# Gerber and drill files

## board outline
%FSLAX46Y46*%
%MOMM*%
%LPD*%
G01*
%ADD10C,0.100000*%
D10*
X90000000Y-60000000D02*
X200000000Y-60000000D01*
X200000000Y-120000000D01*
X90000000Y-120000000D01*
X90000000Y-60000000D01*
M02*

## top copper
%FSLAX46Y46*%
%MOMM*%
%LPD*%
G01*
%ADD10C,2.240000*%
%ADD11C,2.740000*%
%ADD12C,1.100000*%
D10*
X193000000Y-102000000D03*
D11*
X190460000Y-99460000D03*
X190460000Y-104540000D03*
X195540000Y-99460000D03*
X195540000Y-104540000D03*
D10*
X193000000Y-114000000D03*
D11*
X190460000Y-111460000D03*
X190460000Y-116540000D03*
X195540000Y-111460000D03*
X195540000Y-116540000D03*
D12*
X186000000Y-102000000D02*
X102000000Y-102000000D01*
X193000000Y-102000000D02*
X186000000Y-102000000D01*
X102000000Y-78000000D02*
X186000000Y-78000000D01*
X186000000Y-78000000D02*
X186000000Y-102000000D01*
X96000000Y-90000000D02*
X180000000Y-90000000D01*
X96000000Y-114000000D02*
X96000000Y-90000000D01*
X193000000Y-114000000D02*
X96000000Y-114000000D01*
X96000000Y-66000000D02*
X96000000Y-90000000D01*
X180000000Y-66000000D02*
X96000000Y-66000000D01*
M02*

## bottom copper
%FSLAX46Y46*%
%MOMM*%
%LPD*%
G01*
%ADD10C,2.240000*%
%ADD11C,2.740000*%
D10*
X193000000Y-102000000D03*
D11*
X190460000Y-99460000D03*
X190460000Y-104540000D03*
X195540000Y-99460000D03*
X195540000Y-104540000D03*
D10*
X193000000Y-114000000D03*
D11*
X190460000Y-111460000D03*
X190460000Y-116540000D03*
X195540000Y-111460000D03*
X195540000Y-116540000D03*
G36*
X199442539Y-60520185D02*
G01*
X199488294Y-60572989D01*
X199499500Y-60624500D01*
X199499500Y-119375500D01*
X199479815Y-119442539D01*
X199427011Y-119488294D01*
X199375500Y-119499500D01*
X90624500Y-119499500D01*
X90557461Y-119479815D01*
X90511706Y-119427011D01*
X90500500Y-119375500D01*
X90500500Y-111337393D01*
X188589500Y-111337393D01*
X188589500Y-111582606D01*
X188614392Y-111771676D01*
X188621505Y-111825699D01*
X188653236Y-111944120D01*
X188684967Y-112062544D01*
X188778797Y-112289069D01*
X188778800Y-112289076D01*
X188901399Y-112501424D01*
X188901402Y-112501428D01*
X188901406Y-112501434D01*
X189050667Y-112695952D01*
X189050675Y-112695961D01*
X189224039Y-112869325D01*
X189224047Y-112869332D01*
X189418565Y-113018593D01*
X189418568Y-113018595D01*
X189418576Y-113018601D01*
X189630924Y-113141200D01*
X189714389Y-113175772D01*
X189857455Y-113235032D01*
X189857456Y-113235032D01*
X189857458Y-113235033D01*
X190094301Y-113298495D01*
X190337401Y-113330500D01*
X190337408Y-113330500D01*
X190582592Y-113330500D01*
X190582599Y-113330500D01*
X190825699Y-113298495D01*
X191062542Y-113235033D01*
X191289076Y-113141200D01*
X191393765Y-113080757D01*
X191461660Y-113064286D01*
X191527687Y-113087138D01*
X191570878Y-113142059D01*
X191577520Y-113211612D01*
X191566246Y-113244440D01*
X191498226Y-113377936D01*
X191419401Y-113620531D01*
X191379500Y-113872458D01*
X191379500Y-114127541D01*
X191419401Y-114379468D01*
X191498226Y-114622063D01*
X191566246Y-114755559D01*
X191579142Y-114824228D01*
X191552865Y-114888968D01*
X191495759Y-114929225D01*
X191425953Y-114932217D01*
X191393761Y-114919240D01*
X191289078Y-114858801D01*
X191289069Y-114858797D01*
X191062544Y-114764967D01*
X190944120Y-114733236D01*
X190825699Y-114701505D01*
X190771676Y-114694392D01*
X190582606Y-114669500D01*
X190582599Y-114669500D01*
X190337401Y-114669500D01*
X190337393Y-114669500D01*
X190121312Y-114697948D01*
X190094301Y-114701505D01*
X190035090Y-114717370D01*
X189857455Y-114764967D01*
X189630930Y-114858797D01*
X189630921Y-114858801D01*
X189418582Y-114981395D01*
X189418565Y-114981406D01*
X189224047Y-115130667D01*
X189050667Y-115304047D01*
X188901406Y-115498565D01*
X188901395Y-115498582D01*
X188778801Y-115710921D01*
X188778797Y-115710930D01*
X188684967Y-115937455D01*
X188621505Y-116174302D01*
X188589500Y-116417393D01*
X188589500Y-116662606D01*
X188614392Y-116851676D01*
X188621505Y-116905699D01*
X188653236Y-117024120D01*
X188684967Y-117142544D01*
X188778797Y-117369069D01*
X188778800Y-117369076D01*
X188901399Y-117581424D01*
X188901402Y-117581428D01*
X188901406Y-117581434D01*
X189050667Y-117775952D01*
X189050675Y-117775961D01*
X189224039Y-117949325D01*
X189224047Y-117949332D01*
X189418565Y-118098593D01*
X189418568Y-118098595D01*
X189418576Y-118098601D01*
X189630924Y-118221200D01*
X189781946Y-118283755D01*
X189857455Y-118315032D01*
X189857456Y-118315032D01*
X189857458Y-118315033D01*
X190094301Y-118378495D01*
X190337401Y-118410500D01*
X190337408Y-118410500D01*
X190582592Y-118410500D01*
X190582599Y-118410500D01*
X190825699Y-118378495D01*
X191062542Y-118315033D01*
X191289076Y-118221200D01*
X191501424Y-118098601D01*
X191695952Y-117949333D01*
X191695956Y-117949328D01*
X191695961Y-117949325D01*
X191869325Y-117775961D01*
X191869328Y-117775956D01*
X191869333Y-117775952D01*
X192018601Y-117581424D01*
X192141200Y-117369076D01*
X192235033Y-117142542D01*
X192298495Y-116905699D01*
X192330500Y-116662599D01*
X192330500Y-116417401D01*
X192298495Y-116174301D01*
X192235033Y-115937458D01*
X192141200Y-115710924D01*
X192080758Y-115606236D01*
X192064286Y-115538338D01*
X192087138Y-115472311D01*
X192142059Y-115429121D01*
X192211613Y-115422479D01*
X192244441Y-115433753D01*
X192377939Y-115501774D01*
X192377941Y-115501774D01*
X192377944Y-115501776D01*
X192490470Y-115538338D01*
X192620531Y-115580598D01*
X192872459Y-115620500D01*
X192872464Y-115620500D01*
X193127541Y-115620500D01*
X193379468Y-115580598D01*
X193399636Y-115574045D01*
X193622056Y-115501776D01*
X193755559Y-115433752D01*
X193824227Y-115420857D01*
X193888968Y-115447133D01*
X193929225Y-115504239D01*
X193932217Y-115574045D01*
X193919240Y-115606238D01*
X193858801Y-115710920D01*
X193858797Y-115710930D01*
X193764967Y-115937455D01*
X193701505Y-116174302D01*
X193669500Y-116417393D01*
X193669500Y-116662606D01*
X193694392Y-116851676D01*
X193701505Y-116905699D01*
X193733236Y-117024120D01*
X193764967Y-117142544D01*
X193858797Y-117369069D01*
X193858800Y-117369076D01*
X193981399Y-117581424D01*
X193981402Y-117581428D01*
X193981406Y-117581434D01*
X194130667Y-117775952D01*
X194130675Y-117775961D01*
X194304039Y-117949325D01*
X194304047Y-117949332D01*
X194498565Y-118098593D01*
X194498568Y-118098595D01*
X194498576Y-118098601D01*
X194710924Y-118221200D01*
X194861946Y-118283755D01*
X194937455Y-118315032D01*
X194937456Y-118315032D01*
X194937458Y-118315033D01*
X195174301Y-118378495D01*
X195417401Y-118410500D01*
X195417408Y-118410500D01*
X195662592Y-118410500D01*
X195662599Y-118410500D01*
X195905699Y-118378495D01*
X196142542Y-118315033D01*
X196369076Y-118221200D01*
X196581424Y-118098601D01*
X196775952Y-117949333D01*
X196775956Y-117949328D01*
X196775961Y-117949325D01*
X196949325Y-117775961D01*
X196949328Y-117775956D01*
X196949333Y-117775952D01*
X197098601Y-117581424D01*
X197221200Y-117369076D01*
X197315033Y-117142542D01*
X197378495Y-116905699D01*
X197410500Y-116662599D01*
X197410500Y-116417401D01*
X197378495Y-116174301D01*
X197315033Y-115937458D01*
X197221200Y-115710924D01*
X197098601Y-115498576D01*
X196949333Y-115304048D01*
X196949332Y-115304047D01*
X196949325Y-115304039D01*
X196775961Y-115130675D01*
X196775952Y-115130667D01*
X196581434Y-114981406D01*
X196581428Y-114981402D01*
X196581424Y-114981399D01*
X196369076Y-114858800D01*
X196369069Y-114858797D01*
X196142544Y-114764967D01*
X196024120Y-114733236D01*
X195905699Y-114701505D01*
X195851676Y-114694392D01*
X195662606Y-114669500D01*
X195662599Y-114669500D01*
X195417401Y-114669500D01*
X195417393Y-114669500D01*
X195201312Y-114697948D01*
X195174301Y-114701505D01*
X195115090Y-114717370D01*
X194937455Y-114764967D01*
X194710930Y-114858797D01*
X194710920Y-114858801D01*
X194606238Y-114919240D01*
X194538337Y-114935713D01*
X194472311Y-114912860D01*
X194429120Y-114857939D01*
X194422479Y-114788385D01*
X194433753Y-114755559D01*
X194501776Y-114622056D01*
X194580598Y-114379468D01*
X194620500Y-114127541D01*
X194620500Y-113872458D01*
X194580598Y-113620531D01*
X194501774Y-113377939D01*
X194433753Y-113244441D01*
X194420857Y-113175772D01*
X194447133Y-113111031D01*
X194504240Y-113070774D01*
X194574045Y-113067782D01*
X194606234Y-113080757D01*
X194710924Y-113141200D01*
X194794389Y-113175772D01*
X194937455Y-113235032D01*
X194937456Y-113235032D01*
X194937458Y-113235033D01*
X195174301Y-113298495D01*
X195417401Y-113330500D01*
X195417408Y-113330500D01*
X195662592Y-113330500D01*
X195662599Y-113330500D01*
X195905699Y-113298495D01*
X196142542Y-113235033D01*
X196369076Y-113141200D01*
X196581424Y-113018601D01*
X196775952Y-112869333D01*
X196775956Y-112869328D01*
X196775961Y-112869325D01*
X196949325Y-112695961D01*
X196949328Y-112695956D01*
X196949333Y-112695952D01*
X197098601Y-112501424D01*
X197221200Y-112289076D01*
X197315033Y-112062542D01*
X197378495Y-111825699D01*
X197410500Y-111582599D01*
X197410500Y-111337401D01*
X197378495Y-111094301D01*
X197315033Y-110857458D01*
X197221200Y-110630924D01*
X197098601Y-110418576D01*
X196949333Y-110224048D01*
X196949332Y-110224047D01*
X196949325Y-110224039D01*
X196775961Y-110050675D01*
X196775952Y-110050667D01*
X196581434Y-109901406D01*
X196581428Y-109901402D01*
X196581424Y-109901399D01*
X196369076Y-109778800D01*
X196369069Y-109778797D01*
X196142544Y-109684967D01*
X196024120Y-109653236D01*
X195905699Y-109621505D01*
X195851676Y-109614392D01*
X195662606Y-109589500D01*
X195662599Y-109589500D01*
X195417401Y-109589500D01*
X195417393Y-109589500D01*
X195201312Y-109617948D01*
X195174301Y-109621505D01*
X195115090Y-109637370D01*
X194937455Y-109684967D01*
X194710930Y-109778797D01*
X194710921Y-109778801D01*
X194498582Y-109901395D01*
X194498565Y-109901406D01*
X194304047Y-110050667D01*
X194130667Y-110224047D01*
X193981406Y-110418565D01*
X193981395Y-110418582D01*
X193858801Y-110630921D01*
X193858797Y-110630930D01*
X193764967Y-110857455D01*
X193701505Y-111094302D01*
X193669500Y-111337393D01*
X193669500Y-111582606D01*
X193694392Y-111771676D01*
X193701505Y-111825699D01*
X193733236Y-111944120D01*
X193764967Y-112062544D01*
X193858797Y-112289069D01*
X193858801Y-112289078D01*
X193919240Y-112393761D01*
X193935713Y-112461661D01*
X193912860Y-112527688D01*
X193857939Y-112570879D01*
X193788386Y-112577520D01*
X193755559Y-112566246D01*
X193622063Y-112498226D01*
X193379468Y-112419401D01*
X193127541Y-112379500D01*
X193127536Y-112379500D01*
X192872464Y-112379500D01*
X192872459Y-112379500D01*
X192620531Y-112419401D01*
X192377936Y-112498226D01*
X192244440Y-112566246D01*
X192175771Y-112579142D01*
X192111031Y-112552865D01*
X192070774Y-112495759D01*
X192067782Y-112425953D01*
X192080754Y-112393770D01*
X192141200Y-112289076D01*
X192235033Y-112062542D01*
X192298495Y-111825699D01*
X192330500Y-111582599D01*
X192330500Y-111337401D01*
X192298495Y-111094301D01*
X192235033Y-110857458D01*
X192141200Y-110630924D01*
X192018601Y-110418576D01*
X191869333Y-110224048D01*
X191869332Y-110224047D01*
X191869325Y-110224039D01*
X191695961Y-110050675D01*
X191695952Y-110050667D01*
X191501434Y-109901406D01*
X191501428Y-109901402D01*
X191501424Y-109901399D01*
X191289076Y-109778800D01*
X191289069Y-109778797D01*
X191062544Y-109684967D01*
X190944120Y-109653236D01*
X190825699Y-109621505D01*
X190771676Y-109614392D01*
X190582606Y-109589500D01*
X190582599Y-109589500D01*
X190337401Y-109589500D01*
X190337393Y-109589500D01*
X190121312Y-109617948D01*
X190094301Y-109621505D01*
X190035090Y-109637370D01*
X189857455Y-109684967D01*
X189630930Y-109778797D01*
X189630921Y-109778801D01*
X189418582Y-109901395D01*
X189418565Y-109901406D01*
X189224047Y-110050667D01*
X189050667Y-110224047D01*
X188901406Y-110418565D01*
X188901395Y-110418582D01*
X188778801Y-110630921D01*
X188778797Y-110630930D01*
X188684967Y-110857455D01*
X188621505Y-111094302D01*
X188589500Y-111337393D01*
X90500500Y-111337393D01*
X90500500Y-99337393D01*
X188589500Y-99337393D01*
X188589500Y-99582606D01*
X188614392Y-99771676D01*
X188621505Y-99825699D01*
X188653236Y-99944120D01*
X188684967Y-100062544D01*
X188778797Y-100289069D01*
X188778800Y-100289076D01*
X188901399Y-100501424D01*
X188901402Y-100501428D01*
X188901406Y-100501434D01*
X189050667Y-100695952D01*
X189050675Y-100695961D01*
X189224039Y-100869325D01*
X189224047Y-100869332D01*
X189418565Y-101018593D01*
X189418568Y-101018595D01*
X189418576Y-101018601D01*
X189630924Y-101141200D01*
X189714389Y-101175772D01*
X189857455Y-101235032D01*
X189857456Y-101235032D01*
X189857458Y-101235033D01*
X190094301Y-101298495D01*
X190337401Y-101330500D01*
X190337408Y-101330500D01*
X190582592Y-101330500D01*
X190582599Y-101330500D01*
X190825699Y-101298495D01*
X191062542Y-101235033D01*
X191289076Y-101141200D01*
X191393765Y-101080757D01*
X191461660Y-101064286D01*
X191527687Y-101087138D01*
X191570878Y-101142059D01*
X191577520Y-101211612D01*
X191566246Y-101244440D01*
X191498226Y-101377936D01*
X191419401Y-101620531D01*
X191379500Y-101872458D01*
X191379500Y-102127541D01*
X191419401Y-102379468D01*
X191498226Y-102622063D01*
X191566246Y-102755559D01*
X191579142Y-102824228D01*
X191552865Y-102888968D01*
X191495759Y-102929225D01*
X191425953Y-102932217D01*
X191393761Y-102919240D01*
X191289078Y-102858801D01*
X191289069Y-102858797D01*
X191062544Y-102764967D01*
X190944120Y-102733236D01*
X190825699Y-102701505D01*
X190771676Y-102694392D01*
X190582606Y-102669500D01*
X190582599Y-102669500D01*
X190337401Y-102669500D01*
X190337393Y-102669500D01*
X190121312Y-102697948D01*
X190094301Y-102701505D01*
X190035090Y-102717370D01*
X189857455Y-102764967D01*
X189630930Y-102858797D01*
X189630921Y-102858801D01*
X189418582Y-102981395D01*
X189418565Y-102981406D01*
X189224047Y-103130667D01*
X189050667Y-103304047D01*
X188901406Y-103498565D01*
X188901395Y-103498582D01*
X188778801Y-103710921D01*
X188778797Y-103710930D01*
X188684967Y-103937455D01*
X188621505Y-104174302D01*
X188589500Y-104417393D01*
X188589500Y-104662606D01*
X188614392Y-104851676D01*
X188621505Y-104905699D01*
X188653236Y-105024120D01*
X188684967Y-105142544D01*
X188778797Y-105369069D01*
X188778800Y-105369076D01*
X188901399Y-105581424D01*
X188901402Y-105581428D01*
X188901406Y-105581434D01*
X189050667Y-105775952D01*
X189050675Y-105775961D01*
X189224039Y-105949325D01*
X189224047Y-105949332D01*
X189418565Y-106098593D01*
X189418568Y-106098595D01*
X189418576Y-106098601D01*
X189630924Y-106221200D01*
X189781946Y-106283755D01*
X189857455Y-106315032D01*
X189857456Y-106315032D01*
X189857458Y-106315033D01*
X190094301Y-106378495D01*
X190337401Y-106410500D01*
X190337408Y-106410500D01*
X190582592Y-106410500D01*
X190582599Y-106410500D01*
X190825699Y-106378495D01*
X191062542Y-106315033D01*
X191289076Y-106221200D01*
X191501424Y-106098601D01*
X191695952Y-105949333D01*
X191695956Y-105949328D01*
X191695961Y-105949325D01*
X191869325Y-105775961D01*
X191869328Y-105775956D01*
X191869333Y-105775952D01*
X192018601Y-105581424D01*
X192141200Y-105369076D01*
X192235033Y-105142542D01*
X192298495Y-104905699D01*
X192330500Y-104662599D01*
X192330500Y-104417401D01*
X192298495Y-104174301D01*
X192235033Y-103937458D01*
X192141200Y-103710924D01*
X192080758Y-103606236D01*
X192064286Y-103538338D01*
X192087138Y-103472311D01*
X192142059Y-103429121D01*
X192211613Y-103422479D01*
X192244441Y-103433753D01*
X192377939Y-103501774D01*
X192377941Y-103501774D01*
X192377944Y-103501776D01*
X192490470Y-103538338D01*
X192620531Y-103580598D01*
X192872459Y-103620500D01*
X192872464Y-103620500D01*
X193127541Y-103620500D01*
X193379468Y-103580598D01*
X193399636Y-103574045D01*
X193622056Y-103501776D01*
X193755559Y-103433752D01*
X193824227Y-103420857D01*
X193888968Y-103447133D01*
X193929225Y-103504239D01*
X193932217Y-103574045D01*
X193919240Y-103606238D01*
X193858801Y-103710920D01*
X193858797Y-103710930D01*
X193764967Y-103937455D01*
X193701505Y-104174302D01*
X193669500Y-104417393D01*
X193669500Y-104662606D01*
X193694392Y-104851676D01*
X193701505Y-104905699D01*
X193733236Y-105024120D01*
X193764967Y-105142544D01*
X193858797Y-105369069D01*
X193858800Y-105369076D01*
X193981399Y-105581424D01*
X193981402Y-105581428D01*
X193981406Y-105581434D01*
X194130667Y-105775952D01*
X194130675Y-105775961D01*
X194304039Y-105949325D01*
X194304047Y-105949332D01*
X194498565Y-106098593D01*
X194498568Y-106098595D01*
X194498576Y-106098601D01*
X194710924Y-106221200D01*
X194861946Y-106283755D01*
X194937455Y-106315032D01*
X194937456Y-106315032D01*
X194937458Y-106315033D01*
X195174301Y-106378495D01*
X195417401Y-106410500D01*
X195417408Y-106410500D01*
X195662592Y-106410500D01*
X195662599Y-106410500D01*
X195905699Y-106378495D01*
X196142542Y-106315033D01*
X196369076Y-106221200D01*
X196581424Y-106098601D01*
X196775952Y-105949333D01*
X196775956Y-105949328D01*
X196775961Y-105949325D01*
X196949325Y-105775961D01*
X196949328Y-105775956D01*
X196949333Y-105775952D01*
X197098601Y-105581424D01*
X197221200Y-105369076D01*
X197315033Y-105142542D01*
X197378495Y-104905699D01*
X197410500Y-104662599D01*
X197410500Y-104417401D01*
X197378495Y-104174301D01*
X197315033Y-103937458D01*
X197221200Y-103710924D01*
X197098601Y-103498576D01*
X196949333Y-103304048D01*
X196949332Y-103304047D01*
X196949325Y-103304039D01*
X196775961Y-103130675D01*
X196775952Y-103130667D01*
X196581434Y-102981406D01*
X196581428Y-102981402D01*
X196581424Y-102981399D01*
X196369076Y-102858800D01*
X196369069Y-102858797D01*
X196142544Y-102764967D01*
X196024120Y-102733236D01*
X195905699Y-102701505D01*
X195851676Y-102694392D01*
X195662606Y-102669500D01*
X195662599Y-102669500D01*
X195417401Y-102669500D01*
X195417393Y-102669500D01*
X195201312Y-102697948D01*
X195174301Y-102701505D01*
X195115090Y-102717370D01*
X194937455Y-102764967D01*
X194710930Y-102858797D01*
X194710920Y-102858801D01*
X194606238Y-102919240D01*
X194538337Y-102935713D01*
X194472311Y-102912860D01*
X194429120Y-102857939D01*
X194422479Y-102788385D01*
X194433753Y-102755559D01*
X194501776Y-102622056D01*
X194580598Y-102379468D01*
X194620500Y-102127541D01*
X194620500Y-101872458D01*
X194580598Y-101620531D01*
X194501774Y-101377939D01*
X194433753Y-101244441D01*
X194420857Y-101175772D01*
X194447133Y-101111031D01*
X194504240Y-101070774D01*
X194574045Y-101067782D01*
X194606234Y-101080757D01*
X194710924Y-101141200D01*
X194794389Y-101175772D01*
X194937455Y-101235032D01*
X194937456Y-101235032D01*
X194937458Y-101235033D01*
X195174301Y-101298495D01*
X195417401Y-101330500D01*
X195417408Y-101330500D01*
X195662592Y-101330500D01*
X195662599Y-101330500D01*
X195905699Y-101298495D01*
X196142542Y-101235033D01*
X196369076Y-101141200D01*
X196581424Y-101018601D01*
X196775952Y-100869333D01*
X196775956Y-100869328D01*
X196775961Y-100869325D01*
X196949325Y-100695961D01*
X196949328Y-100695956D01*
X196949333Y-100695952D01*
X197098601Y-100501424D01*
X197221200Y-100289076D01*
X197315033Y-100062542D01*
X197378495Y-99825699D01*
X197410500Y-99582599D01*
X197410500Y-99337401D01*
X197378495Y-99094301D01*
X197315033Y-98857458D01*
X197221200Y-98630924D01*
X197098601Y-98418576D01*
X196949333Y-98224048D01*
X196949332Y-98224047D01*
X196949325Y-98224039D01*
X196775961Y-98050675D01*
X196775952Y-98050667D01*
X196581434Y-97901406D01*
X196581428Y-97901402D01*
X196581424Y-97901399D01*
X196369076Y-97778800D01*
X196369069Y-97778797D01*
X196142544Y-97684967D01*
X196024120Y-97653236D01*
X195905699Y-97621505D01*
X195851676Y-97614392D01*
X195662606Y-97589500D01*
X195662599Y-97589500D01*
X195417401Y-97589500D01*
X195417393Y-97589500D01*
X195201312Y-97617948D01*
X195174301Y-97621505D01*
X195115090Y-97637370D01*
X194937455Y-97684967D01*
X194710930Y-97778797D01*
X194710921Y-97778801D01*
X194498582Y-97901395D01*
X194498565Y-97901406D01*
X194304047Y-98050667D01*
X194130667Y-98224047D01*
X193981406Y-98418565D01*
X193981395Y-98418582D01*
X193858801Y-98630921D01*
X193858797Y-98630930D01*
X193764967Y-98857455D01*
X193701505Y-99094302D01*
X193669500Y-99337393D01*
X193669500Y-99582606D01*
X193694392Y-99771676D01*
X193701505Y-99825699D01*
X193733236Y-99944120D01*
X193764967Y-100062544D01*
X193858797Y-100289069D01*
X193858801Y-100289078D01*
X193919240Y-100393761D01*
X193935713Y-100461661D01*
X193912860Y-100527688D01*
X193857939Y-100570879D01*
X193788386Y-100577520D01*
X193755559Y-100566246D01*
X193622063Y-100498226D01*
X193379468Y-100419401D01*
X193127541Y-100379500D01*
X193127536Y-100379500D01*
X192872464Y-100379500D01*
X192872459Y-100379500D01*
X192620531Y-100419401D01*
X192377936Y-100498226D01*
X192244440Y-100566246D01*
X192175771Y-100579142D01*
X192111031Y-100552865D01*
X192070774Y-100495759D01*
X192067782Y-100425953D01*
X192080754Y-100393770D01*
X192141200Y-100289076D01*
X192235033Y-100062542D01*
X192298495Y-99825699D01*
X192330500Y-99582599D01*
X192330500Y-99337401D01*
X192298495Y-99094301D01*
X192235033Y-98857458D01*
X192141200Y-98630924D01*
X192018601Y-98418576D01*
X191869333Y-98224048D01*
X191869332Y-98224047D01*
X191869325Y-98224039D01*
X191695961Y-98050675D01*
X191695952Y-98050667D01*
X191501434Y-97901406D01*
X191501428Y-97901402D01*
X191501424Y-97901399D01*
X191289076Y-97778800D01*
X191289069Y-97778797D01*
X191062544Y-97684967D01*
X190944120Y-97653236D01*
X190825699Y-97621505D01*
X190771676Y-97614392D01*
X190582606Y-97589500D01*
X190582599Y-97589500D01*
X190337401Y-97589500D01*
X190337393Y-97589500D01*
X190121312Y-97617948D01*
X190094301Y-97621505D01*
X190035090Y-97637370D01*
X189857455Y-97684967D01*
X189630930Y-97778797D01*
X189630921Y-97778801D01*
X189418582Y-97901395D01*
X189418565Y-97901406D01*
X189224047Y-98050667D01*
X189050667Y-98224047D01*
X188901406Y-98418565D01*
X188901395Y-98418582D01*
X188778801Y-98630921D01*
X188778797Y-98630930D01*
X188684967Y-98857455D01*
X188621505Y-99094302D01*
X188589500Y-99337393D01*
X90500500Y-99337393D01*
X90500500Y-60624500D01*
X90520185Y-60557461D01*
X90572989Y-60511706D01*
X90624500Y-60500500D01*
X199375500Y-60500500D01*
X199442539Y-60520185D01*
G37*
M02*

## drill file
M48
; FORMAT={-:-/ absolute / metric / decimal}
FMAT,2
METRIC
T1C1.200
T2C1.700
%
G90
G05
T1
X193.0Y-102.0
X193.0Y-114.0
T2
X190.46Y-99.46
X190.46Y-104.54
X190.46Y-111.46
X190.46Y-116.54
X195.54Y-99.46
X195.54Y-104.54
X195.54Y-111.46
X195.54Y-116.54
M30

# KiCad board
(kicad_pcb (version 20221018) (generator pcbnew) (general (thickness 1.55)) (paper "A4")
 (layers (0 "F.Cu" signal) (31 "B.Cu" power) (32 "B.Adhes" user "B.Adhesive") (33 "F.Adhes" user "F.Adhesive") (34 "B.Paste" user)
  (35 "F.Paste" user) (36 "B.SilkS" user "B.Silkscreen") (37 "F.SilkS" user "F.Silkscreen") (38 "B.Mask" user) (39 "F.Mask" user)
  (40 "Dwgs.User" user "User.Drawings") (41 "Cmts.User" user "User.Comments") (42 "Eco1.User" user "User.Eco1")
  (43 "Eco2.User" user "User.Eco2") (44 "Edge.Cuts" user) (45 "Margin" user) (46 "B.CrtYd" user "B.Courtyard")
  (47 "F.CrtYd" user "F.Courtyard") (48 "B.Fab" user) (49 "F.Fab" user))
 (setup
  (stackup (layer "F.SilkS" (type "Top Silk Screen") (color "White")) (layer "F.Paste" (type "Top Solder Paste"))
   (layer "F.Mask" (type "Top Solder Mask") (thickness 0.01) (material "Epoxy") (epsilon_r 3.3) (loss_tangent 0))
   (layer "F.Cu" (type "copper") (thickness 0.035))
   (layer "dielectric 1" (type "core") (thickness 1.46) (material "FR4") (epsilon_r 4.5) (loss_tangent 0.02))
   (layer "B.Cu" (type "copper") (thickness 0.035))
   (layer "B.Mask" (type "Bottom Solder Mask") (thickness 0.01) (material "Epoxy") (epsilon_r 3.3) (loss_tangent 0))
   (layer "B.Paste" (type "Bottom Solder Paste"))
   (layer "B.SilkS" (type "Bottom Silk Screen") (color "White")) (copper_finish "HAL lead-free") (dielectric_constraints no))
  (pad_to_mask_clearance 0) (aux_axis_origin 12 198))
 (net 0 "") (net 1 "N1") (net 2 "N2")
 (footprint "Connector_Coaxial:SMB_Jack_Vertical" (layer "F.Cu") (at 193 102)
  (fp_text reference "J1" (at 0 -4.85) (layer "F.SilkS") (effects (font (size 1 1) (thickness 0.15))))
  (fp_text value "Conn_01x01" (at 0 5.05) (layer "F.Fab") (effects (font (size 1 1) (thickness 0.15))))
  (pad "1" thru_hole circle (at 0 0) (size 2.24 2.24) (drill 1.2) (layers "*.Cu" "*.Mask") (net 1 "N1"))
  (pad "2" thru_hole circle (at -2.54 -2.54) (size 2.74 2.74) (drill 1.7) (layers "*.Cu" "*.Mask"))
  (pad "2" thru_hole circle (at -2.54 2.54) (size 2.74 2.74) (drill 1.7) (layers "*.Cu" "*.Mask"))
  (pad "2" thru_hole circle (at 2.54 -2.54) (size 2.74 2.74) (drill 1.7) (layers "*.Cu" "*.Mask"))
  (pad "2" thru_hole circle (at 2.54 2.54) (size 2.74 2.74) (drill 1.7) (layers "*.Cu" "*.Mask")))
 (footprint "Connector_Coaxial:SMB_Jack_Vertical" (layer "F.Cu") (at 193 114)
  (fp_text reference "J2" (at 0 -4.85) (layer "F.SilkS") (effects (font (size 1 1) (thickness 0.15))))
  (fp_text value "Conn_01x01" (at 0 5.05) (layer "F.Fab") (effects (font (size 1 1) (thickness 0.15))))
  (pad "1" thru_hole circle (at 0 0) (size 2.24 2.24) (drill 1.2) (layers "*.Cu" "*.Mask") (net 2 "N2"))
  (pad "2" thru_hole circle (at -2.54 -2.54) (size 2.74 2.74) (drill 1.7) (layers "*.Cu" "*.Mask"))
  (pad "2" thru_hole circle (at -2.54 2.54) (size 2.74 2.74) (drill 1.7) (layers "*.Cu" "*.Mask"))
  (pad "2" thru_hole circle (at 2.54 -2.54) (size 2.74 2.74) (drill 1.7) (layers "*.Cu" "*.Mask"))
  (pad "2" thru_hole circle (at 2.54 2.54) (size 2.74 2.74) (drill 1.7) (layers "*.Cu" "*.Mask")))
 (gr_rect (start 90 60) (end 200 120) (stroke (width 0.1) (type default)) (fill none) (layer "Edge.Cuts"))
 (segment (start 186 102) (end 102 102) (width 1.1) (layer "F.Cu") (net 1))
 (segment (start 193 102) (end 186 102) (width 1.1) (layer "F.Cu") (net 1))
 (segment (start 102 78) (end 186 78) (width 1.1) (layer "F.Cu") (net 1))
 (segment (start 186 78) (end 186 102) (width 1.1) (layer "F.Cu") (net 1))
 (segment (start 96 90) (end 180 90) (width 1.1) (layer "F.Cu") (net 2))
 (segment (start 96 114) (end 96 90) (width 1.1) (layer "F.Cu") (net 2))
 (segment (start 193 114) (end 96 114) (width 1.1) (layer "F.Cu") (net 2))
 (segment (start 96 66) (end 96 90) (width 1.1) (layer "F.Cu") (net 2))
 (segment (start 180 66) (end 96 66) (width 1.1) (layer "F.Cu") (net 2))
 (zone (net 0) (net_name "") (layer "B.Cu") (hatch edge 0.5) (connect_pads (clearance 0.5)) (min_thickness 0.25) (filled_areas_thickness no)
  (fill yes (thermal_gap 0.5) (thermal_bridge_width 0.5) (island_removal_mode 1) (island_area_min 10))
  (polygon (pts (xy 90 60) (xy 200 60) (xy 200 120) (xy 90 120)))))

